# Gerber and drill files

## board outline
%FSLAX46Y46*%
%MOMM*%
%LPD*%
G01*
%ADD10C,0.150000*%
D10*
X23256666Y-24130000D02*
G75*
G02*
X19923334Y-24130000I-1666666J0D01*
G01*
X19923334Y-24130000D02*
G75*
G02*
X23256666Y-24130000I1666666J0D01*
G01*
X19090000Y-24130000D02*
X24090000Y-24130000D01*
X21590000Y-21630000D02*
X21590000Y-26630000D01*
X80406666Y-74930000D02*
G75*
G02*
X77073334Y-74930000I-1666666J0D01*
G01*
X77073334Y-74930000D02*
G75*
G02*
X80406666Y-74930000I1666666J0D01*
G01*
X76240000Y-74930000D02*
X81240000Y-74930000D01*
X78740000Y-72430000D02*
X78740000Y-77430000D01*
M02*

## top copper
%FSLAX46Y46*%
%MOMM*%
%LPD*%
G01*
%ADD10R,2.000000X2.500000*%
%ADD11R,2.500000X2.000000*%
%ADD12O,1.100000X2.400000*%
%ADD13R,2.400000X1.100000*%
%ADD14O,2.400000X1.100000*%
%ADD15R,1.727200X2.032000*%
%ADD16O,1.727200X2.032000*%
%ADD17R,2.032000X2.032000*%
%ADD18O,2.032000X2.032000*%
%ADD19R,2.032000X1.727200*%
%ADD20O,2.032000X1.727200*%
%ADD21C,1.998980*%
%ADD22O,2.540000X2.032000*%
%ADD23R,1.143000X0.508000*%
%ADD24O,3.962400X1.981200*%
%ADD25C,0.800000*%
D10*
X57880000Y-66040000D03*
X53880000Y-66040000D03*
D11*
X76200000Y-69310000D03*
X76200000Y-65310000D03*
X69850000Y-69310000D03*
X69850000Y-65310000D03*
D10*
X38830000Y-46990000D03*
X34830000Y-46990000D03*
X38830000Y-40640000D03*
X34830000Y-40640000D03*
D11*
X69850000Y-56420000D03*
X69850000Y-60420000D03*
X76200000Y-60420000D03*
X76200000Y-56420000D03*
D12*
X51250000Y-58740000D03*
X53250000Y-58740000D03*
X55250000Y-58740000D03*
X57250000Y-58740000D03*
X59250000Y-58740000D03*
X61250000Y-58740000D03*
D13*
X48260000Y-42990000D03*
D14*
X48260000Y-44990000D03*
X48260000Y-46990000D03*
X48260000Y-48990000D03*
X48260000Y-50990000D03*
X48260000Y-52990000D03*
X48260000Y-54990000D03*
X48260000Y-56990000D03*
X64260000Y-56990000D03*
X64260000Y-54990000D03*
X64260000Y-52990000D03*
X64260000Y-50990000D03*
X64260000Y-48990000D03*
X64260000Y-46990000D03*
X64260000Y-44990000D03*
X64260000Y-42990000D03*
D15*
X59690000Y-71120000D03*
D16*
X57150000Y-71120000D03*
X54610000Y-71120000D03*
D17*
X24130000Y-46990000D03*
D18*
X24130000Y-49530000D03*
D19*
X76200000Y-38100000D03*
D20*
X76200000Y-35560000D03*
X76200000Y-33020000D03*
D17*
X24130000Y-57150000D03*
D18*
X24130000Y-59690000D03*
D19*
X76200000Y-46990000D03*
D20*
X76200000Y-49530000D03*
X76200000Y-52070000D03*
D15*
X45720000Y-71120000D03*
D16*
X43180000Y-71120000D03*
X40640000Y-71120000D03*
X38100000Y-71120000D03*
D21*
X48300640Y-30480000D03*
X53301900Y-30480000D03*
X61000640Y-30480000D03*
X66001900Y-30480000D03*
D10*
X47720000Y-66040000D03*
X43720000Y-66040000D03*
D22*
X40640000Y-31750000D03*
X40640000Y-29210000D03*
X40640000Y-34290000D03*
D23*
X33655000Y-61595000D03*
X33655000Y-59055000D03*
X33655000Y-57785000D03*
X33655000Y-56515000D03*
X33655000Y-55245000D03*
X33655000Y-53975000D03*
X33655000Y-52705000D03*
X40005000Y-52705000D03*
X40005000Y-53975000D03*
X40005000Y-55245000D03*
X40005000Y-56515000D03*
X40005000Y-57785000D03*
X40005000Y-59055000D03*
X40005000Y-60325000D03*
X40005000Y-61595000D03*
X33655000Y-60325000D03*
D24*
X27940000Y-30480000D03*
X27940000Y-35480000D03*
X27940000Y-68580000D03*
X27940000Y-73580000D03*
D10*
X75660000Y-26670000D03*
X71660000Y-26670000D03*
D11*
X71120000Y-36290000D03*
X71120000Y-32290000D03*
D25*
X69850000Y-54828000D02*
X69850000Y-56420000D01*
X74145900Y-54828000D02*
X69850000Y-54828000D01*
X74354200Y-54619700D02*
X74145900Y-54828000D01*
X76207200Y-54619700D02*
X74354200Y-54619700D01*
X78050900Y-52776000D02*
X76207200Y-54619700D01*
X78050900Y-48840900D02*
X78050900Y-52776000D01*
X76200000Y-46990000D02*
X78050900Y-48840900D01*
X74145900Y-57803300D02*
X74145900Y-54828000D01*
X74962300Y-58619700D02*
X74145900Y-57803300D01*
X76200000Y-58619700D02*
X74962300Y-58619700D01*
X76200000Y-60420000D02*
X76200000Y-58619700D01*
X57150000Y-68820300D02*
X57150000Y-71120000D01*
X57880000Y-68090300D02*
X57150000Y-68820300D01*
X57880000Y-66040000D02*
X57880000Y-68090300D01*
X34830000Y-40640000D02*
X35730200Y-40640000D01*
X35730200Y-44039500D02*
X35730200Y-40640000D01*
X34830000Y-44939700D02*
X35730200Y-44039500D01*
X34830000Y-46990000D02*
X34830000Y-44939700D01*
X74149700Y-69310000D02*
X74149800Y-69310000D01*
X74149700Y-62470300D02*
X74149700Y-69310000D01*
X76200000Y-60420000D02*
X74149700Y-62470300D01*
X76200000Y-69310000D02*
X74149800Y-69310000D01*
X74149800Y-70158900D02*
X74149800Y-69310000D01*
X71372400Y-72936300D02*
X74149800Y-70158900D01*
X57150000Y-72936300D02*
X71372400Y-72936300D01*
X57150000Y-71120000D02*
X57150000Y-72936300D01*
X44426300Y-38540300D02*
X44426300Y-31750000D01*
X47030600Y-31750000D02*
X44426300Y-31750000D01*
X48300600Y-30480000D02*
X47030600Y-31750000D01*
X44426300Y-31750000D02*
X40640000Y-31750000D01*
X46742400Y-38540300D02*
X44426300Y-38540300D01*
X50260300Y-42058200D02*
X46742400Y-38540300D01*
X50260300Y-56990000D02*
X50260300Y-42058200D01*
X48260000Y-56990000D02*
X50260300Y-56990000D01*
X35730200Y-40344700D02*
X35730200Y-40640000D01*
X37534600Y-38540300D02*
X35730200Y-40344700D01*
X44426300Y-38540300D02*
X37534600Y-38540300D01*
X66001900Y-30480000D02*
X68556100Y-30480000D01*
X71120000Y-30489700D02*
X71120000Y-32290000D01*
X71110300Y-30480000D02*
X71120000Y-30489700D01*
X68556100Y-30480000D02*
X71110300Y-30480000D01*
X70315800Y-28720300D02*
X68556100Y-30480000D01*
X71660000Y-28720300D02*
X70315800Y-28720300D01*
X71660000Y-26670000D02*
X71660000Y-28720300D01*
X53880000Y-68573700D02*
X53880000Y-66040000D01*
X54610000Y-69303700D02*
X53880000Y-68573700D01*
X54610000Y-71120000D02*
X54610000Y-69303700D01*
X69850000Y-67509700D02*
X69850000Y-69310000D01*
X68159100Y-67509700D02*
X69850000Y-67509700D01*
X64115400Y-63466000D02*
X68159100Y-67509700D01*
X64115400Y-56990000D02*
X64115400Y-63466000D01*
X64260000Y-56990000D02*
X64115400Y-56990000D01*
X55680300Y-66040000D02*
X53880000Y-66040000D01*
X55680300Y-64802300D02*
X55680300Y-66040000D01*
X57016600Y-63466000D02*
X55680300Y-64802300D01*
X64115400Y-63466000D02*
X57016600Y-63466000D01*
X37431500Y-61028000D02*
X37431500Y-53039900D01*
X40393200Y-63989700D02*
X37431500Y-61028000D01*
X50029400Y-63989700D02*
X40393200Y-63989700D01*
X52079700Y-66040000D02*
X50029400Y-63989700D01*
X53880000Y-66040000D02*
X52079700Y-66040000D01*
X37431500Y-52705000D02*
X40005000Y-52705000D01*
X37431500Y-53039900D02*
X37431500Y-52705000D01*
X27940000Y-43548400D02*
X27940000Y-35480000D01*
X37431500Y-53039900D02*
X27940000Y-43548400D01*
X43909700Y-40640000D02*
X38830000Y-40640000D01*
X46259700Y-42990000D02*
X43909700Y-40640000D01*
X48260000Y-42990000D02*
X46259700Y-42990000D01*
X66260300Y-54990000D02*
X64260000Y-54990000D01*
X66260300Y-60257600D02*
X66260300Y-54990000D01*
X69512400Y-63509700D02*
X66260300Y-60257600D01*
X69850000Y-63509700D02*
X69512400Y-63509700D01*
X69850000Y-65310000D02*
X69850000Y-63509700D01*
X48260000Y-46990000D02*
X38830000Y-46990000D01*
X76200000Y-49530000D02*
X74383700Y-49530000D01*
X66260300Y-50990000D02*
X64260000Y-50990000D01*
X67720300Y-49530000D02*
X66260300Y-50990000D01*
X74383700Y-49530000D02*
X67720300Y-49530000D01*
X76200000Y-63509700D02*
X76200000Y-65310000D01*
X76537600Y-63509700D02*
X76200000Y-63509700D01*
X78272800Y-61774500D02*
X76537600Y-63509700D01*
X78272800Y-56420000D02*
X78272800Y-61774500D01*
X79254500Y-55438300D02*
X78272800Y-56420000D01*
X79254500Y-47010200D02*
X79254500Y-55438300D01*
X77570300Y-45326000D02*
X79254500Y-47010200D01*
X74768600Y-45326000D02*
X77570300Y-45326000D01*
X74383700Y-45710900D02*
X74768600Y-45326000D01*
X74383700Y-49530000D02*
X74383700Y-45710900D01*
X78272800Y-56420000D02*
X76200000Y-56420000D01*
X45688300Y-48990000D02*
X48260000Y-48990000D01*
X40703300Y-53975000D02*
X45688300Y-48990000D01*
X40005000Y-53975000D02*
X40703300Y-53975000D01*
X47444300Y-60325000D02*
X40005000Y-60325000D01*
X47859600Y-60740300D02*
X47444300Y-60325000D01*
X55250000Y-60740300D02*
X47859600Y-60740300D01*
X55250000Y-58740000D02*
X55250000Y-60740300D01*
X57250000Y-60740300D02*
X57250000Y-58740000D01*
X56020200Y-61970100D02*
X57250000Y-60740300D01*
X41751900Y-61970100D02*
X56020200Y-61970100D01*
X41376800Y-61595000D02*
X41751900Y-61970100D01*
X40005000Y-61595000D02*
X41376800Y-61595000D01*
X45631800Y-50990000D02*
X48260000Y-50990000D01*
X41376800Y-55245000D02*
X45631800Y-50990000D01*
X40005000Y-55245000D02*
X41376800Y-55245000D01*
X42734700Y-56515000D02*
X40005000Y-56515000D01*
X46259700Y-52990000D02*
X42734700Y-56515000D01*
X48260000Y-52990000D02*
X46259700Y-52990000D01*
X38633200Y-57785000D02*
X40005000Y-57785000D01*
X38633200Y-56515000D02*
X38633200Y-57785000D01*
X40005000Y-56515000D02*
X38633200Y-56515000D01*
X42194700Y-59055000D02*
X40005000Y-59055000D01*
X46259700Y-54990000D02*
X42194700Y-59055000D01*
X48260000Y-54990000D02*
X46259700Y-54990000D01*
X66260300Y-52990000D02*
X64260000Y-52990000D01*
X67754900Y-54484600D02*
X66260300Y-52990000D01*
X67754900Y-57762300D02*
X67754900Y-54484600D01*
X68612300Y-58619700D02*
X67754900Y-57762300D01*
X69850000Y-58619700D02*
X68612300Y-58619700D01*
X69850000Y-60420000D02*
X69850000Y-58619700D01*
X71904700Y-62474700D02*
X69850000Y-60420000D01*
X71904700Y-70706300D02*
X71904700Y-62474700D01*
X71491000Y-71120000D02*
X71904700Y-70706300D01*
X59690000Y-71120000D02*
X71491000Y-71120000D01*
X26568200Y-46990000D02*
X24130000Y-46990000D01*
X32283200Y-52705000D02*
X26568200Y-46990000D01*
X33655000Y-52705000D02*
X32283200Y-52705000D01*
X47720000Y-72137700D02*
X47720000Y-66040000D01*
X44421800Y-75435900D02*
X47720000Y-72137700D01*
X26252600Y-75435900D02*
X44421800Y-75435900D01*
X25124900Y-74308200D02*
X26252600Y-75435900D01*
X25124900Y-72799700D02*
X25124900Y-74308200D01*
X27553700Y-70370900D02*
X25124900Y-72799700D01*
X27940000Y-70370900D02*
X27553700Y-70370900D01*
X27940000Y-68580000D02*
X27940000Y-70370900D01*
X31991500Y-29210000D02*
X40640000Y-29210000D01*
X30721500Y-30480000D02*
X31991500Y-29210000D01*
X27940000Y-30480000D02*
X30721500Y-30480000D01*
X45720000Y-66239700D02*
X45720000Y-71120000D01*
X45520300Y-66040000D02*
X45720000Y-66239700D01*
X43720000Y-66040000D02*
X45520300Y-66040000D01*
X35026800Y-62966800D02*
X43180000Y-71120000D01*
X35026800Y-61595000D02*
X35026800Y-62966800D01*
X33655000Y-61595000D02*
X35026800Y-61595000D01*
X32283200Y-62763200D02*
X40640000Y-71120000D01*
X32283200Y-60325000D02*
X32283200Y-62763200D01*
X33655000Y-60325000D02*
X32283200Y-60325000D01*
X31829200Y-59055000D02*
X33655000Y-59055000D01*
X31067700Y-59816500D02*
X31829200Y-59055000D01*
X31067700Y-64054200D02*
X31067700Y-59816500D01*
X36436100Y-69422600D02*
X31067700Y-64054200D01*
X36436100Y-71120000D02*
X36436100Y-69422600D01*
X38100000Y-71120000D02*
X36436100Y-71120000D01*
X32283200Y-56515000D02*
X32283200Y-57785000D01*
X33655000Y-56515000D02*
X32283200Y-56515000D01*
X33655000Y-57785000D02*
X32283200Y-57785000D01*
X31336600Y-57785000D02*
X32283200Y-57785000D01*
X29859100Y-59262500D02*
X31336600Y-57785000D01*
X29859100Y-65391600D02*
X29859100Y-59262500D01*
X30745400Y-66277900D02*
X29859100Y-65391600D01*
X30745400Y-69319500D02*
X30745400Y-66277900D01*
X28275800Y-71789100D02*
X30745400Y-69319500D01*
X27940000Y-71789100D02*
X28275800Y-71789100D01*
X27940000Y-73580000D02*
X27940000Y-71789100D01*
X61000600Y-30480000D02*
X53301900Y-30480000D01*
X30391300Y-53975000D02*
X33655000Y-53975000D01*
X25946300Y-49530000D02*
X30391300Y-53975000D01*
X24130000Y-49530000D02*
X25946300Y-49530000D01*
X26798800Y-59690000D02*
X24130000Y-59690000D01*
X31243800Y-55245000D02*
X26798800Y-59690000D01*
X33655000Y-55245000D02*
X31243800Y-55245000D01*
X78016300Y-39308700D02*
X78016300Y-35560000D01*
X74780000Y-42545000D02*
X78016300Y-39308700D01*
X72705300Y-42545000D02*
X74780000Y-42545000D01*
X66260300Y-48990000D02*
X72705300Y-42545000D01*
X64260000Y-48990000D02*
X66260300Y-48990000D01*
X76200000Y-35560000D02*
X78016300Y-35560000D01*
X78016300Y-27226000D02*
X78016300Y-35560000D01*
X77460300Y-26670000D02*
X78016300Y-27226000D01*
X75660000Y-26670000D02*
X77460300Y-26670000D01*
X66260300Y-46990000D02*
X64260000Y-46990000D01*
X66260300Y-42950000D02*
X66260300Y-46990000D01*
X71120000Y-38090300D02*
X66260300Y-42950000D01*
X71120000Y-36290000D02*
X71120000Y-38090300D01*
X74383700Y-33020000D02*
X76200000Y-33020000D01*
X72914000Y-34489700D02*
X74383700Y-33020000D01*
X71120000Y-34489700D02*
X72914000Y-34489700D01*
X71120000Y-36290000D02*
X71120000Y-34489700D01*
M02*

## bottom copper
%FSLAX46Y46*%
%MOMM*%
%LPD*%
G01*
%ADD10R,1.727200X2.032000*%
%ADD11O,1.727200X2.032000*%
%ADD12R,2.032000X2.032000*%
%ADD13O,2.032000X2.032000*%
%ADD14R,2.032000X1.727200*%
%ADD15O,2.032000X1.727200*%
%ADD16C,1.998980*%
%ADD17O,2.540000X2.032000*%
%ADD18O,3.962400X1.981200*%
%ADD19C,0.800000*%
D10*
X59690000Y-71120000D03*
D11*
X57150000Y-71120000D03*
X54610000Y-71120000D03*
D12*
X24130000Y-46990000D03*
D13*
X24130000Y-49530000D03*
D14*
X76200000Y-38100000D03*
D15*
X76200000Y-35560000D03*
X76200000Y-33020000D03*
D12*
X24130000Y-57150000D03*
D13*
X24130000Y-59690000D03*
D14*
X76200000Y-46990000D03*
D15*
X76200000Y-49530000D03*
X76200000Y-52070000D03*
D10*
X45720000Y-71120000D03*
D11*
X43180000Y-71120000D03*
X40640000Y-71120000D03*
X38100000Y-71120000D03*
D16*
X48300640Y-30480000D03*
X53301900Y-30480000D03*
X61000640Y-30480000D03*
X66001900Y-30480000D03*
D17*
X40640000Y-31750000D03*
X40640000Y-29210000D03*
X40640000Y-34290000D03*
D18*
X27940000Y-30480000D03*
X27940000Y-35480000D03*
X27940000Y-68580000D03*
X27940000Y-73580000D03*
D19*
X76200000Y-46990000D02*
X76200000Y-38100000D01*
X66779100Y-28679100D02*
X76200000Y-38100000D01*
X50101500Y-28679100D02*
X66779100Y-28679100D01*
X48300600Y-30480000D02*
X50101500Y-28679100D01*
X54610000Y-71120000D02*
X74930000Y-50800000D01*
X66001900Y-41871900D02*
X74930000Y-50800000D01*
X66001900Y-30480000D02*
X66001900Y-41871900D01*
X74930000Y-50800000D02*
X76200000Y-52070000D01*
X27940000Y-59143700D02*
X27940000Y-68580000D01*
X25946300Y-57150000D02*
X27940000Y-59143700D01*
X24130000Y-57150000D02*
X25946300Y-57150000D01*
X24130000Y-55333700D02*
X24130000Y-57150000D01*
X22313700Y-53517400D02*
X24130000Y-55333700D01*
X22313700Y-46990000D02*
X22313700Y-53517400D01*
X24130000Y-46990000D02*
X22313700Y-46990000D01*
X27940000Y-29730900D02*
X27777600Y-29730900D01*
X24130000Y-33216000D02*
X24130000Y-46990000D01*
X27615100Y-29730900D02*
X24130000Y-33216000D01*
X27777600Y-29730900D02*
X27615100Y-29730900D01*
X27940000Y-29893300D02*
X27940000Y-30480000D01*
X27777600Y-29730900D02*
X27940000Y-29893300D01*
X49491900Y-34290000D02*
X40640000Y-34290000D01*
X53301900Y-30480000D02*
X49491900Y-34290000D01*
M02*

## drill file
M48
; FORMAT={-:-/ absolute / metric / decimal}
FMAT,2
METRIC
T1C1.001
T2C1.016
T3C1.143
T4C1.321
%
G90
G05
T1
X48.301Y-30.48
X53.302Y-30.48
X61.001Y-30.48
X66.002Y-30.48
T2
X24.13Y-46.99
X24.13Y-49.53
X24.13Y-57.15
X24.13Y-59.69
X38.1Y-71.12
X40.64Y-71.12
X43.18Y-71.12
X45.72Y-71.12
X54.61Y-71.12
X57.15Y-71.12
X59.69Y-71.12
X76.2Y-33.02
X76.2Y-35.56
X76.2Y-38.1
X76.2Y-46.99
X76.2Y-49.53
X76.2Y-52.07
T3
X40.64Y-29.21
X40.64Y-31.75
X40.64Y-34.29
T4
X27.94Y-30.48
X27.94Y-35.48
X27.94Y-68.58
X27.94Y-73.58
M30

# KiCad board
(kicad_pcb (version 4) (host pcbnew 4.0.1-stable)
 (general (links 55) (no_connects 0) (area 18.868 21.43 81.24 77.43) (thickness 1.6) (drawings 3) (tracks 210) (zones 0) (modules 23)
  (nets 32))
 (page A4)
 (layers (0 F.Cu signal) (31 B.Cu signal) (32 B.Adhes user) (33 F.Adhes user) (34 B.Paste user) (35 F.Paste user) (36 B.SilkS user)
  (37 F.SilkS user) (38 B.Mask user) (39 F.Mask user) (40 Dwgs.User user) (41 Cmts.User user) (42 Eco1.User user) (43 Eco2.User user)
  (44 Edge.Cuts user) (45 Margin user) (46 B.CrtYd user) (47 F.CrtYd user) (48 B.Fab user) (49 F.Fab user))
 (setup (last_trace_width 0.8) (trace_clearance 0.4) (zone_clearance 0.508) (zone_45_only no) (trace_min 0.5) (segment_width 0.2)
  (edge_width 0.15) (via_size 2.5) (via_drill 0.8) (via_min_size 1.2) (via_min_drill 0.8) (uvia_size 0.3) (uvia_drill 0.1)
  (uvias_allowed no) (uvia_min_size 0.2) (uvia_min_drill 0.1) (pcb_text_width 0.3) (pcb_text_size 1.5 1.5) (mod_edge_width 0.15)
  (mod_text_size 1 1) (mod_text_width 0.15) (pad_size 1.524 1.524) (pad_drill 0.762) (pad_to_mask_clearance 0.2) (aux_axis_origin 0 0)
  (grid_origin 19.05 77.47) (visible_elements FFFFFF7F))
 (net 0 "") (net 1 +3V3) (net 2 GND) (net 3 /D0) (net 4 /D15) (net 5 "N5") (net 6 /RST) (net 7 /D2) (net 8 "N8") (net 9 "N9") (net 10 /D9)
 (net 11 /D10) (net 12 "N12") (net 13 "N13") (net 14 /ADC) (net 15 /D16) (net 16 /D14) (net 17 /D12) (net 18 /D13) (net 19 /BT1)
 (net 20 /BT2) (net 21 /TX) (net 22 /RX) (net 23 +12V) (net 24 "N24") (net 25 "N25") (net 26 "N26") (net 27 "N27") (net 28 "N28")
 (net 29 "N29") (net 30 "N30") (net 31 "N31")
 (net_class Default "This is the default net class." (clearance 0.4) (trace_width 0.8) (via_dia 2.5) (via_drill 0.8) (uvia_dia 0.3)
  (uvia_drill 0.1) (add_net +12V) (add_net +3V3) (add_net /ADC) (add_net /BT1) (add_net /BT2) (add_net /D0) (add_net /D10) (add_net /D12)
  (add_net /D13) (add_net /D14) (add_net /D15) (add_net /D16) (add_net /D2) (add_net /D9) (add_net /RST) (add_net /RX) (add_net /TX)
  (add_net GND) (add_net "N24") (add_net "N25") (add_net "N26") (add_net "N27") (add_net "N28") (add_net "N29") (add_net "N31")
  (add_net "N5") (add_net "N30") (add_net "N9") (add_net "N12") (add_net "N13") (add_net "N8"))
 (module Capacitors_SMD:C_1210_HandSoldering (layer F.Cu) (at 55.88 66.04 180)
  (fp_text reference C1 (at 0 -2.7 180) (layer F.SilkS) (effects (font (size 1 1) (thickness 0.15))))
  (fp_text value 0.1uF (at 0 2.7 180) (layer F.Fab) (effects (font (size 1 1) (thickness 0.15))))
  (pad 1 smd rect (at -2 0 180) (size 2 2.5) (layers F.Cu F.Paste F.Mask) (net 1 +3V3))
  (pad 2 smd rect (at 2 0 180) (size 2 2.5) (layers F.Cu F.Paste F.Mask) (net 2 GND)))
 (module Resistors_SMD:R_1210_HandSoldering (layer F.Cu) (at 76.2 67.31 90)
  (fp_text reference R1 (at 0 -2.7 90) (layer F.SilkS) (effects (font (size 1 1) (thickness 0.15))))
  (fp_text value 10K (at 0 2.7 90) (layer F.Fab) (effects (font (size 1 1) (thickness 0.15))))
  (pad 1 smd rect (at -2 0 90) (size 2 2.5) (layers F.Cu F.Paste F.Mask) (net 1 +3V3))
  (pad 2 smd rect (at 2 0 90) (size 2 2.5) (layers F.Cu F.Paste F.Mask) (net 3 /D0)))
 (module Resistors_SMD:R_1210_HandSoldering (layer F.Cu) (at 69.85 67.31 90)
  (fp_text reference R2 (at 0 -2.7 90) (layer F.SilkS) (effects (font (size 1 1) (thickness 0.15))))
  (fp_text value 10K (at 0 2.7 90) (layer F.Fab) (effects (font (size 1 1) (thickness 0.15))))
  (pad 1 smd rect (at -2 0 90) (size 2 2.5) (layers F.Cu F.Paste F.Mask) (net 2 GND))
  (pad 2 smd rect (at 2 0 90) (size 2 2.5) (layers F.Cu F.Paste F.Mask) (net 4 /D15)))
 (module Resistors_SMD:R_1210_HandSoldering (layer F.Cu) (at 36.83 46.99 180)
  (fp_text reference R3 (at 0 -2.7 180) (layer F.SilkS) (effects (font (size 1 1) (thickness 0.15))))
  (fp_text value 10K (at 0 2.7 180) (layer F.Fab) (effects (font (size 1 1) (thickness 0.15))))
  (pad 1 smd rect (at -2 0 180) (size 2 2.5) (layers F.Cu F.Paste F.Mask) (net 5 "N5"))
  (pad 2 smd rect (at 2 0 180) (size 2 2.5) (layers F.Cu F.Paste F.Mask) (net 1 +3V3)))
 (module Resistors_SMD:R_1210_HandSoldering (layer F.Cu) (at 36.83 40.64 180)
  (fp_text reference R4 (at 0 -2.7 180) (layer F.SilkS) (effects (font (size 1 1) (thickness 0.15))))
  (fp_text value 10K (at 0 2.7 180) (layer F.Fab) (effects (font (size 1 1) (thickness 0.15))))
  (pad 1 smd rect (at -2 0 180) (size 2 2.5) (layers F.Cu F.Paste F.Mask) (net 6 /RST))
  (pad 2 smd rect (at 2 0 180) (size 2 2.5) (layers F.Cu F.Paste F.Mask) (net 1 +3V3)))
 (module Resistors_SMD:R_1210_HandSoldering (layer F.Cu) (at 69.85 58.42 270)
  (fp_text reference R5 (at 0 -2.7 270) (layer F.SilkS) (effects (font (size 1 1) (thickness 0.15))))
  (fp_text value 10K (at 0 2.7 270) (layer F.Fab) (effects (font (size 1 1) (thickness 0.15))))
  (pad 1 smd rect (at -2 0 270) (size 2 2.5) (layers F.Cu F.Paste F.Mask) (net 1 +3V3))
  (pad 2 smd rect (at 2 0 270) (size 2 2.5) (layers F.Cu F.Paste F.Mask) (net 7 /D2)))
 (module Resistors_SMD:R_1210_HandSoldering (layer F.Cu) (at 76.2 58.42 90)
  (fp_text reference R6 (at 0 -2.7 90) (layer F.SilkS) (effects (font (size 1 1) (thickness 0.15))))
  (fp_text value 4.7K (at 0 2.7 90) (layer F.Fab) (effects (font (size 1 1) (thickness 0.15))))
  (pad 1 smd rect (at -2 0 90) (size 2 2.5) (layers F.Cu F.Paste F.Mask) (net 1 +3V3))
  (pad 2 smd rect (at 2 0 90) (size 2 2.5) (layers F.Cu F.Paste F.Mask) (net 3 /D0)))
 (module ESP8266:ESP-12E (layer F.Cu) (at 48.26 42.99)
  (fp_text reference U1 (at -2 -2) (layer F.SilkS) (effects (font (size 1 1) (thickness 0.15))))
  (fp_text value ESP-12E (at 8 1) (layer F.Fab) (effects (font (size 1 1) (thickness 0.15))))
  (pad 9 smd oval (at 2.99 15.75 90) (size 2.4 1.1) (layers F.Cu F.Paste F.Mask) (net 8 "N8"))
  (pad 10 smd oval (at 4.99 15.75 90) (size 2.4 1.1) (layers F.Cu F.Paste F.Mask) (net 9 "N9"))
  (pad 11 smd oval (at 6.99 15.75 90) (size 2.4 1.1) (layers F.Cu F.Paste F.Mask) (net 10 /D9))
  (pad 12 smd oval (at 8.99 15.75 90) (size 2.4 1.1) (layers F.Cu F.Paste F.Mask) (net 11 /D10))
  (pad 13 smd oval (at 10.99 15.75 90) (size 2.4 1.1) (layers F.Cu F.Paste F.Mask) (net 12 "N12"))
  (pad 14 smd oval (at 12.99 15.75 90) (size 2.4 1.1) (layers F.Cu F.Paste F.Mask) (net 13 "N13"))
  (pad 1 smd rect (at 0 0) (size 2.4 1.1) (layers F.Cu F.Paste F.Mask) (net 6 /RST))
  (pad 2 smd oval (at 0 2) (size 2.4 1.1) (layers F.Cu F.Paste F.Mask) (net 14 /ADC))
  (pad 3 smd oval (at 0 4) (size 2.4 1.1) (layers F.Cu F.Paste F.Mask) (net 5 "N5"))
  (pad 4 smd oval (at 0 6) (size 2.4 1.1) (layers F.Cu F.Paste F.Mask) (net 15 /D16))
  (pad 5 smd oval (at 0 8) (size 2.4 1.1) (layers F.Cu F.Paste F.Mask) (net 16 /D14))
  (pad 6 smd oval (at 0 10) (size 2.4 1.1) (layers F.Cu F.Paste F.Mask) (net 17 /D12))
  (pad 7 smd oval (at 0 12) (size 2.4 1.1) (layers F.Cu F.Paste F.Mask) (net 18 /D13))
  (pad 8 smd oval (at 0 14) (size 2.4 1.1) (layers F.Cu F.Paste F.Mask) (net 1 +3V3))
  (pad 15 smd oval (at 16 14) (size 2.4 1.1) (layers F.Cu F.Paste F.Mask) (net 2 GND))
  (pad 16 smd oval (at 16 12) (size 2.4 1.1) (layers F.Cu F.Paste F.Mask) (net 4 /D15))
  (pad 17 smd oval (at 16 10) (size 2.4 1.1) (layers F.Cu F.Paste F.Mask) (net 7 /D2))
  (pad 18 smd oval (at 16 8) (size 2.4 1.1) (layers F.Cu F.Paste F.Mask) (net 3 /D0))
  (pad 19 smd oval (at 16 6) (size 2.4 1.1) (layers F.Cu F.Paste F.Mask) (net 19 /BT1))
  (pad 20 smd oval (at 16 4) (size 2.4 1.1) (layers F.Cu F.Paste F.Mask) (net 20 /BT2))
  (pad 21 smd oval (at 16 2) (size 2.4 1.1) (layers F.Cu F.Paste F.Mask) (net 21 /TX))
  (pad 22 smd oval (at 16 0) (size 2.4 1.1) (layers F.Cu F.Paste F.Mask) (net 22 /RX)))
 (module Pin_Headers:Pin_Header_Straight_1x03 (layer F.Cu) (at 59.69 71.12 270)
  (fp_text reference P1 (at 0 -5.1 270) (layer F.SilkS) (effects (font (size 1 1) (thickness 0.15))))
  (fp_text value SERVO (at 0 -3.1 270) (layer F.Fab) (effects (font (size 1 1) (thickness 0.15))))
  (pad 1 thru_hole rect (at 0 0 270) (size 2.032 1.7272) (drill 1.016) (layers *.Cu *.Mask F.SilkS) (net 7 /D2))
  (pad 2 thru_hole oval (at 0 2.54 270) (size 2.032 1.7272) (drill 1.016) (layers *.Cu *.Mask F.SilkS) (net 1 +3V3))
  (pad 3 thru_hole oval (at 0 5.08 270) (size 2.032 1.7272) (drill 1.016) (layers *.Cu *.Mask F.SilkS) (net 2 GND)))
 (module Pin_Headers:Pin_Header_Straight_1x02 (layer F.Cu) (at 24.13 46.99)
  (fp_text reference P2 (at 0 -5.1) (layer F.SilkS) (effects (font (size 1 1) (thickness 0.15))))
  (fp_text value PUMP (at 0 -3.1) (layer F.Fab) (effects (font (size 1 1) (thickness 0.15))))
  (pad 1 thru_hole rect (at 0 0) (size 2.032 2.032) (drill 1.016) (layers *.Cu *.Mask F.SilkS) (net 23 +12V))
  (pad 2 thru_hole oval (at 0 2.54) (size 2.032 2.032) (drill 1.016) (layers *.Cu *.Mask F.SilkS) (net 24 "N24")))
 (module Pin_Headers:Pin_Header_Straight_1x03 (layer F.Cu) (at 76.2 38.1 180)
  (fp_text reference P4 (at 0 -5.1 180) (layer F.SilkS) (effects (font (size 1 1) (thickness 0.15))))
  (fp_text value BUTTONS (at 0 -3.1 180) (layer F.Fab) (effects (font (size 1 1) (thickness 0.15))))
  (pad 1 thru_hole rect (at 0 0 180) (size 2.032 1.7272) (drill 1.016) (layers *.Cu *.Mask F.SilkS) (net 1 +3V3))
  (pad 2 thru_hole oval (at 0 2.54 180) (size 2.032 1.7272) (drill 1.016) (layers *.Cu *.Mask F.SilkS) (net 19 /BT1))
  (pad 3 thru_hole oval (at 0 5.08 180) (size 2.032 1.7272) (drill 1.016) (layers *.Cu *.Mask F.SilkS) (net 20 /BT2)))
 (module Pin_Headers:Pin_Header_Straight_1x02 (layer F.Cu) (at 24.13 57.15)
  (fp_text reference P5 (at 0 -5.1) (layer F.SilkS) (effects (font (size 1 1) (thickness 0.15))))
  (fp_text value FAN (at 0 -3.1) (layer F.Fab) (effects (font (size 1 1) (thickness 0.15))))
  (pad 1 thru_hole rect (at 0 0) (size 2.032 2.032) (drill 1.016) (layers *.Cu *.Mask F.SilkS) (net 23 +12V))
  (pad 2 thru_hole oval (at 0 2.54) (size 2.032 2.032) (drill 1.016) (layers *.Cu *.Mask F.SilkS) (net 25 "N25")))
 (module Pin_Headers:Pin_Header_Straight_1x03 (layer F.Cu) (at 76.2 46.99)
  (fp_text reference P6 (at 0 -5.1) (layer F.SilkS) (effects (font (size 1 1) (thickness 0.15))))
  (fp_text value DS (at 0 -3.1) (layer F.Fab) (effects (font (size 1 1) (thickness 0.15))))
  (pad 1 thru_hole rect (at 0 0) (size 2.032 1.7272) (drill 1.016) (layers *.Cu *.Mask F.SilkS) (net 1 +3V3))
  (pad 2 thru_hole oval (at 0 2.54) (size 2.032 1.7272) (drill 1.016) (layers *.Cu *.Mask F.SilkS) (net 3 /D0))
  (pad 3 thru_hole oval (at 0 5.08) (size 2.032 1.7272) (drill 1.016) (layers *.Cu *.Mask F.SilkS) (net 2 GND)))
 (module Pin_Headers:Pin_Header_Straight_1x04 (layer F.Cu) (at 45.72 71.12 270)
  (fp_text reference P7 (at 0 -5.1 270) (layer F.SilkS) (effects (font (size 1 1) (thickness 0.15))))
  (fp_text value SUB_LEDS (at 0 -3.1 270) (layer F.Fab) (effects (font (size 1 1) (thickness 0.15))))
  (pad 1 thru_hole rect (at 0 0 270) (size 2.032 1.7272) (drill 1.016) (layers *.Cu *.Mask F.SilkS) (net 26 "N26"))
  (pad 2 thru_hole oval (at 0 2.54 270) (size 2.032 1.7272) (drill 1.016) (layers *.Cu *.Mask F.SilkS) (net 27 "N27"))
  (pad 3 thru_hole oval (at 0 5.08 270) (size 2.032 1.7272) (drill 1.016) (layers *.Cu *.Mask F.SilkS) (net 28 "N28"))
  (pad 4 thru_hole oval (at 0 7.62 270) (size 2.032 1.7272) (drill 1.016) (layers *.Cu *.Mask F.SilkS) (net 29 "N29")))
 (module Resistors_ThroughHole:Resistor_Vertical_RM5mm (layer F.Cu) (at 50.8 30.48)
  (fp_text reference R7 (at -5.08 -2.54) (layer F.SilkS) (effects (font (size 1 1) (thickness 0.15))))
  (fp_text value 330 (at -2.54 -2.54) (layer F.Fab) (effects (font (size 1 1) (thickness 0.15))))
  (pad 1 thru_hole circle (at -2.49936 0) (size 1.99898 1.99898) (drill 1.00076) (layers *.Cu *.SilkS *.Mask) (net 1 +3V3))
  (pad 2 thru_hole circle (at 2.5019 0) (size 1.99898 1.99898) (drill 1.00076) (layers *.Cu *.SilkS *.Mask) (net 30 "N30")))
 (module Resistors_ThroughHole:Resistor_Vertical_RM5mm (layer F.Cu) (at 63.5 30.48)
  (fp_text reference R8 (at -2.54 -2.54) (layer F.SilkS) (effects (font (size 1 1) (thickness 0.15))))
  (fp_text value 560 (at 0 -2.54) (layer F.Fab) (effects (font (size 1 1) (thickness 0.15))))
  (pad 1 thru_hole circle (at -2.49936 0) (size 1.99898 1.99898) (drill 1.00076) (layers *.Cu *.SilkS *.Mask) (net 30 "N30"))
  (pad 2 thru_hole circle (at 2.5019 0) (size 1.99898 1.99898) (drill 1.00076) (layers *.Cu *.SilkS *.Mask) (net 2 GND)))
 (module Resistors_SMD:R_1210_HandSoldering (layer F.Cu) (at 45.72 66.04 180)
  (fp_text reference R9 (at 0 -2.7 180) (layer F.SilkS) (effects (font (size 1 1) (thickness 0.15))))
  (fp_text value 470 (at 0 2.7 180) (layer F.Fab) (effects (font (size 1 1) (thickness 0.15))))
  (pad 1 smd rect (at -2 0 180) (size 2 2.5) (layers F.Cu F.Paste F.Mask) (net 23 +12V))
  (pad 2 smd rect (at 2 0 180) (size 2 2.5) (layers F.Cu F.Paste F.Mask) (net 26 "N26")))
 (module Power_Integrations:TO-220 (layer F.Cu) (at 40.64 31.75 90)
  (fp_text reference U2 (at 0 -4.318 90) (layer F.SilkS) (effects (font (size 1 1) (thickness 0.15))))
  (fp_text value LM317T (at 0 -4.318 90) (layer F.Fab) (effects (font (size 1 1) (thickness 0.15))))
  (pad 2 thru_hole oval (at 0 0 90) (size 2.032 2.54) (drill 1.143) (layers *.Cu *.Mask F.SilkS) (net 1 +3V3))
  (pad 3 thru_hole oval (at 2.54 0 90) (size 2.032 2.54) (drill 1.143) (layers *.Cu *.Mask F.SilkS) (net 23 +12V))
  (pad 1 thru_hole oval (at -2.54 0 90) (size 2.032 2.54) (drill 1.143) (layers *.Cu *.Mask F.SilkS) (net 30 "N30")))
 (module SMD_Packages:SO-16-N (layer F.Cu) (at 36.83 57.15 90)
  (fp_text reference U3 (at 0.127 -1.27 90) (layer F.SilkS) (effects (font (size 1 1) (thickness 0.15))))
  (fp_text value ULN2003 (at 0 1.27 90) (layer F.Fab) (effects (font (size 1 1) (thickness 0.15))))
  (pad 16 smd rect (at -4.445 -3.175 90) (size 0.508 1.143) (layers F.Cu F.Paste F.Mask) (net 27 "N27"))
  (pad 14 smd rect (at -1.905 -3.175 90) (size 0.508 1.143) (layers F.Cu F.Paste F.Mask) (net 29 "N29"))
  (pad 13 smd rect (at -0.635 -3.175 90) (size 0.508 1.143) (layers F.Cu F.Paste F.Mask) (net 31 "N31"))
  (pad 12 smd rect (at 0.635 -3.175 90) (size 0.508 1.143) (layers F.Cu F.Paste F.Mask) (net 31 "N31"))
  (pad 11 smd rect (at 1.905 -3.175 90) (size 0.508 1.143) (layers F.Cu F.Paste F.Mask) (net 25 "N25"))
  (pad 10 smd rect (at 3.175 -3.175 90) (size 0.508 1.143) (layers F.Cu F.Paste F.Mask) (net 24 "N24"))
  (pad 9 smd rect (at 4.445 -3.175 90) (size 0.508 1.143) (layers F.Cu F.Paste F.Mask) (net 23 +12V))
  (pad 8 smd rect (at 4.445 3.175 90) (size 0.508 1.143) (layers F.Cu F.Paste F.Mask) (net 2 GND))
  (pad 7 smd rect (at 3.175 3.175 90) (size 0.508 1.143) (layers F.Cu F.Paste F.Mask) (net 15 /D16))
  (pad 6 smd rect (at 1.905 3.175 90) (size 0.508 1.143) (layers F.Cu F.Paste F.Mask) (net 16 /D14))
  (pad 5 smd rect (at 0.635 3.175 90) (size 0.508 1.143) (layers F.Cu F.Paste F.Mask) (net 17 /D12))
  (pad 4 smd rect (at -0.635 3.175 90) (size 0.508 1.143) (layers F.Cu F.Paste F.Mask) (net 17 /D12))
  (pad 3 smd rect (at -1.905 3.175 90) (size 0.508 1.143) (layers F.Cu F.Paste F.Mask) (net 18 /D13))
  (pad 2 smd rect (at -3.175 3.175 90) (size 0.508 1.143) (layers F.Cu F.Paste F.Mask) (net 10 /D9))
  (pad 1 smd rect (at -4.445 3.175 90) (size 0.508 1.143) (layers F.Cu F.Paste F.Mask) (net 11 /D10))
  (pad 15 smd rect (at -3.175 -3.175 90) (size 0.508 1.143) (layers F.Cu F.Paste F.Mask) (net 28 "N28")))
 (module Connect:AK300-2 (layer F.Cu) (at 27.94 30.48 270)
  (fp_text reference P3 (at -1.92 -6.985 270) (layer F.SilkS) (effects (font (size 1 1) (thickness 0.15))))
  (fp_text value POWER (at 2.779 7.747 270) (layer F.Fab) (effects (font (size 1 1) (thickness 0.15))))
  (pad 1 thru_hole oval (at 0 0 270) (size 1.9812 3.9624) (drill 1.3208) (layers *.Cu F.Paste F.SilkS F.Mask) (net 23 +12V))
  (pad 2 thru_hole oval (at 5 0 270) (size 1.9812 3.9624) (drill 1.3208) (layers *.Cu F.Paste F.SilkS F.Mask) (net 2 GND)))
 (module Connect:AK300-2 (layer F.Cu) (at 27.94 68.58 270)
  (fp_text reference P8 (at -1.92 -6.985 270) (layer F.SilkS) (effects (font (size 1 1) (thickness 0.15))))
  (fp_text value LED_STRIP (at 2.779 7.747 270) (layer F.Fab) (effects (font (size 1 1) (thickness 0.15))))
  (pad 1 thru_hole oval (at 0 0 270) (size 1.9812 3.9624) (drill 1.3208) (layers *.Cu F.Paste F.SilkS F.Mask) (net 23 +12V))
  (pad 2 thru_hole oval (at 5 0 270) (size 1.9812 3.9624) (drill 1.3208) (layers *.Cu F.Paste F.SilkS F.Mask) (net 31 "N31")))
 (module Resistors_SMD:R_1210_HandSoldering (layer F.Cu) (at 73.66 26.67 180)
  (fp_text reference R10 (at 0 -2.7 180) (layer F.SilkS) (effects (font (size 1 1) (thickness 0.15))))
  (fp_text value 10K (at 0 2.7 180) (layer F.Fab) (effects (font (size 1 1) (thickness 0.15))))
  (pad 1 smd rect (at -2 0 180) (size 2 2.5) (layers F.Cu F.Paste F.Mask) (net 19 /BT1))
  (pad 2 smd rect (at 2 0 180) (size 2 2.5) (layers F.Cu F.Paste F.Mask) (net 2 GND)))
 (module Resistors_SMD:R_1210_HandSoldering (layer F.Cu) (at 71.12 34.29 90)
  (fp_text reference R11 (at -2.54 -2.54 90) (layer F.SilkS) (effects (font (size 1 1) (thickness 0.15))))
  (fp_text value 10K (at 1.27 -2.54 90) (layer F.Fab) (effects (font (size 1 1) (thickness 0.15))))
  (pad 1 smd rect (at -2 0 90) (size 2 2.5) (layers F.Cu F.Paste F.Mask) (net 20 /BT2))
  (pad 2 smd rect (at 2 0 90) (size 2 2.5) (layers F.Cu F.Paste F.Mask) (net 2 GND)))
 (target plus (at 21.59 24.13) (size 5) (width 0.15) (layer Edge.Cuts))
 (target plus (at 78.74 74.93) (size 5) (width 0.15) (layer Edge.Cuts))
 (segment (start 76.2 46.99) (end 76.2 38.1) (width 0.8) (layer B.Cu) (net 1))
 (segment (start 69.85 54.828) (end 69.85 56.42) (width 0.8) (layer F.Cu) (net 1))
 (segment (start 74.1459 54.828) (end 69.85 54.828) (width 0.8) (layer F.Cu) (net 1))
 (segment (start 74.3542 54.6197) (end 74.1459 54.828) (width 0.8) (layer F.Cu) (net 1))
 (segment (start 76.2072 54.6197) (end 74.3542 54.6197) (width 0.8) (layer F.Cu) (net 1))
 (segment (start 78.0509 52.776) (end 76.2072 54.6197) (width 0.8) (layer F.Cu) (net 1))
 (segment (start 78.0509 48.8409) (end 78.0509 52.776) (width 0.8) (layer F.Cu) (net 1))
 (segment (start 76.2 46.99) (end 78.0509 48.8409) (width 0.8) (layer F.Cu) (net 1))
 (segment (start 74.1459 57.8033) (end 74.1459 54.828) (width 0.8) (layer F.Cu) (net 1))
 (segment (start 74.9623 58.6197) (end 74.1459 57.8033) (width 0.8) (layer F.Cu) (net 1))
 (segment (start 76.2 58.6197) (end 74.9623 58.6197) (width 0.8) (layer F.Cu) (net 1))
 (segment (start 76.2 60.42) (end 76.2 58.6197) (width 0.8) (layer F.Cu) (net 1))
 (segment (start 66.7791 28.6791) (end 76.2 38.1) (width 0.8) (layer B.Cu) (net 1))
 (segment (start 50.1015 28.6791) (end 66.7791 28.6791) (width 0.8) (layer B.Cu) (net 1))
 (segment (start 48.3006 30.48) (end 50.1015 28.6791) (width 0.8) (layer B.Cu) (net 1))
 (segment (start 57.15 68.8203) (end 57.15 71.12) (width 0.8) (layer F.Cu) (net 1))
 (segment (start 57.88 68.0903) (end 57.15 68.8203) (width 0.8) (layer F.Cu) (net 1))
 (segment (start 57.88 66.04) (end 57.88 68.0903) (width 0.8) (layer F.Cu) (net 1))
 (segment (start 34.83 40.64) (end 35.7302 40.64) (width 0.8) (layer F.Cu) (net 1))
 (segment (start 35.7302 44.0395) (end 35.7302 40.64) (width 0.8) (layer F.Cu) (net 1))
 (segment (start 34.83 44.9397) (end 35.7302 44.0395) (width 0.8) (layer F.Cu) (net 1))
 (segment (start 34.83 46.99) (end 34.83 44.9397) (width 0.8) (layer F.Cu) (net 1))
 (segment (start 74.1497 69.31) (end 74.1498 69.31) (width 0.8) (layer F.Cu) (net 1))
 (segment (start 74.1497 62.4703) (end 74.1497 69.31) (width 0.8) (layer F.Cu) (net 1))
 (segment (start 76.2 60.42) (end 74.1497 62.4703) (width 0.8) (layer F.Cu) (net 1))
 (segment (start 76.2 69.31) (end 74.1498 69.31) (width 0.8) (layer F.Cu) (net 1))
 (segment (start 74.1498 70.1589) (end 74.1498 69.31) (width 0.8) (layer F.Cu) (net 1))
 (segment (start 71.3724 72.9363) (end 74.1498 70.1589) (width 0.8) (layer F.Cu) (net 1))
 (segment (start 57.15 72.9363) (end 71.3724 72.9363) (width 0.8) (layer F.Cu) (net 1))
 (segment (start 57.15 71.12) (end 57.15 72.9363) (width 0.8) (layer F.Cu) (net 1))
 (segment (start 44.4263 38.5403) (end 44.4263 31.75) (width 0.8) (layer F.Cu) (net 1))
 (segment (start 47.0306 31.75) (end 44.4263 31.75) (width 0.8) (layer F.Cu) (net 1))
 (segment (start 48.3006 30.48) (end 47.0306 31.75) (width 0.8) (layer F.Cu) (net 1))
 (segment (start 44.4263 31.75) (end 40.64 31.75) (width 0.8) (layer F.Cu) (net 1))
 (segment (start 46.7424 38.5403) (end 44.4263 38.5403) (width 0.8) (layer F.Cu) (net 1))
 (segment (start 50.2603 42.0582) (end 46.7424 38.5403) (width 0.8) (layer F.Cu) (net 1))
 (segment (start 50.2603 56.99) (end 50.2603 42.0582) (width 0.8) (layer F.Cu) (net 1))
 (segment (start 48.26 56.99) (end 50.2603 56.99) (width 0.8) (layer F.Cu) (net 1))
 (segment (start 35.7302 40.3447) (end 35.7302 40.64) (width 0.8) (layer F.Cu) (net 1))
 (segment (start 37.5346 38.5403) (end 35.7302 40.3447) (width 0.8) (layer F.Cu) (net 1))
 (segment (start 44.4263 38.5403) (end 37.5346 38.5403) (width 0.8) (layer F.Cu) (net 1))
 (segment (start 66.0019 30.48) (end 68.5561 30.48) (width 0.8) (layer F.Cu) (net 2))
 (segment (start 71.12 30.4897) (end 71.12 32.29) (width 0.8) (layer F.Cu) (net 2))
 (segment (start 71.1103 30.48) (end 71.12 30.4897) (width 0.8) (layer F.Cu) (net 2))
 (segment (start 68.5561 30.48) (end 71.1103 30.48) (width 0.8) (layer F.Cu) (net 2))
 (segment (start 70.3158 28.7203) (end 68.5561 30.48) (width 0.8) (layer F.Cu) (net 2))
 (segment (start 71.66 28.7203) (end 70.3158 28.7203) (width 0.8) (layer F.Cu) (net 2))
 (segment (start 71.66 26.67) (end 71.66 28.7203) (width 0.8) (layer F.Cu) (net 2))
 (segment (start 53.88 68.5737) (end 53.88 66.04) (width 0.8) (layer F.Cu) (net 2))
 (segment (start 54.61 69.3037) (end 53.88 68.5737) (width 0.8) (layer F.Cu) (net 2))
 (segment (start 54.61 71.12) (end 54.61 69.3037) (width 0.8) (layer F.Cu) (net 2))
 (segment (start 69.85 67.5097) (end 69.85 69.31) (width 0.8) (layer F.Cu) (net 2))
 (segment (start 68.1591 67.5097) (end 69.85 67.5097) (width 0.8) (layer F.Cu) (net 2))
 (segment (start 64.1154 63.466) (end 68.1591 67.5097) (width 0.8) (layer F.Cu) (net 2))
 (segment (start 64.1154 56.99) (end 64.1154 63.466) (width 0.8) (layer F.Cu) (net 2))
 (segment (start 64.26 56.99) (end 64.1154 56.99) (width 0.8) (layer F.Cu) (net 2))
 (segment (start 55.6803 66.04) (end 53.88 66.04) (width 0.8) (layer F.Cu) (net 2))
 (segment (start 55.6803 64.8023) (end 55.6803 66.04) (width 0.8) (layer F.Cu) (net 2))
 (segment (start 57.0166 63.466) (end 55.6803 64.8023) (width 0.8) (layer F.Cu) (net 2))
 (segment (start 64.1154 63.466) (end 57.0166 63.466) (width 0.8) (layer F.Cu) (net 2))
 (segment (start 54.61 71.12) (end 74.93 50.8) (width 0.8) (layer B.Cu) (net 2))
 (segment (start 66.0019 41.8719) (end 74.93 50.8) (width 0.8) (layer B.Cu) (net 2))
 (segment (start 66.0019 30.48) (end 66.0019 41.8719) (width 0.8) (layer B.Cu) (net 2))
 (segment (start 74.93 50.8) (end 76.2 52.07) (width 0.8) (layer B.Cu) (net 2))
 (segment (start 37.4315 61.028) (end 37.4315 53.0399) (width 0.8) (layer F.Cu) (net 2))
 (segment (start 40.3932 63.9897) (end 37.4315 61.028) (width 0.8) (layer F.Cu) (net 2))
 (segment (start 50.0294 63.9897) (end 40.3932 63.9897) (width 0.8) (layer F.Cu) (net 2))
 (segment (start 52.0797 66.04) (end 50.0294 63.9897) (width 0.8) (layer F.Cu) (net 2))
 (segment (start 53.88 66.04) (end 52.0797 66.04) (width 0.8) (layer F.Cu) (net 2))
 (segment (start 37.4315 52.705) (end 40.005 52.705) (width 0.8) (layer F.Cu) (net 2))
 (segment (start 37.4315 53.0399) (end 37.4315 52.705) (width 0.8) (layer F.Cu) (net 2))
 (segment (start 27.94 43.5484) (end 27.94 35.48) (width 0.8) (layer F.Cu) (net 2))
 (segment (start 37.4315 53.0399) (end 27.94 43.5484) (width 0.8) (layer F.Cu) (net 2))
 (segment (start 43.9097 40.64) (end 38.83 40.64) (width 0.8) (layer F.Cu) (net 6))
 (segment (start 46.2597 42.99) (end 43.9097 40.64) (width 0.8) (layer F.Cu) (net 6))
 (segment (start 48.26 42.99) (end 46.2597 42.99) (width 0.8) (layer F.Cu) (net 6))
 (segment (start 66.2603 54.99) (end 64.26 54.99) (width 0.8) (layer F.Cu) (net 4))
 (segment (start 66.2603 60.2576) (end 66.2603 54.99) (width 0.8) (layer F.Cu) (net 4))
 (segment (start 69.5124 63.5097) (end 66.2603 60.2576) (width 0.8) (layer F.Cu) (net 4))
 (segment (start 69.85 63.5097) (end 69.5124 63.5097) (width 0.8) (layer F.Cu) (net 4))
 (segment (start 69.85 65.31) (end 69.85 63.5097) (width 0.8) (layer F.Cu) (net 4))
 (segment (start 48.26 46.99) (end 38.83 46.99) (width 0.8) (layer F.Cu) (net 5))
 (segment (start 76.2 49.53) (end 74.3837 49.53) (width 0.8) (layer F.Cu) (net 3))
 (segment (start 66.2603 50.99) (end 64.26 50.99) (width 0.8) (layer F.Cu) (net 3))
 (segment (start 67.7203 49.53) (end 66.2603 50.99) (width 0.8) (layer F.Cu) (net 3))
 (segment (start 74.3837 49.53) (end 67.7203 49.53) (width 0.8) (layer F.Cu) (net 3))
 (segment (start 76.2 63.5097) (end 76.2 65.31) (width 0.8) (layer F.Cu) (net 3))
 (segment (start 76.5376 63.5097) (end 76.2 63.5097) (width 0.8) (layer F.Cu) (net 3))
 (segment (start 78.2728 61.7745) (end 76.5376 63.5097) (width 0.8) (layer F.Cu) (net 3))
 (segment (start 78.2728 56.42) (end 78.2728 61.7745) (width 0.8) (layer F.Cu) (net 3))
 (segment (start 79.2545 55.4383) (end 78.2728 56.42) (width 0.8) (layer F.Cu) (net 3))
 (segment (start 79.2545 47.0102) (end 79.2545 55.4383) (width 0.8) (layer F.Cu) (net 3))
 (segment (start 77.5703 45.326) (end 79.2545 47.0102) (width 0.8) (layer F.Cu) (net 3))
 (segment (start 74.7686 45.326) (end 77.5703 45.326) (width 0.8) (layer F.Cu) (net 3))
 (segment (start 74.3837 45.7109) (end 74.7686 45.326) (width 0.8) (layer F.Cu) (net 3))
 (segment (start 74.3837 49.53) (end 74.3837 45.7109) (width 0.8) (layer F.Cu) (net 3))
 (segment (start 78.2728 56.42) (end 76.2 56.42) (width 0.8) (layer F.Cu) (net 3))
 (segment (start 45.6883 48.99) (end 48.26 48.99) (width 0.8) (layer F.Cu) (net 15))
 (segment (start 40.7033 53.975) (end 45.6883 48.99) (width 0.8) (layer F.Cu) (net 15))
 (segment (start 40.005 53.975) (end 40.7033 53.975) (width 0.8) (layer F.Cu) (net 15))
 (segment (start 47.4443 60.325) (end 40.005 60.325) (width 0.8) (layer F.Cu) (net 10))
 (segment (start 47.8596 60.7403) (end 47.4443 60.325) (width 0.8) (layer F.Cu) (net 10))
 (segment (start 55.25 60.7403) (end 47.8596 60.7403) (width 0.8) (layer F.Cu) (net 10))
 (segment (start 55.25 58.74) (end 55.25 60.7403) (width 0.8) (layer F.Cu) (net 10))
 (segment (start 57.25 60.7403) (end 57.25 58.74) (width 0.8) (layer F.Cu) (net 11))
 (segment (start 56.0202 61.9701) (end 57.25 60.7403) (width 0.8) (layer F.Cu) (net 11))
 (segment (start 41.7519 61.9701) (end 56.0202 61.9701) (width 0.8) (layer F.Cu) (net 11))
 (segment (start 41.3768 61.595) (end 41.7519 61.9701) (width 0.8) (layer F.Cu) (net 11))
 (segment (start 40.005 61.595) (end 41.3768 61.595) (width 0.8) (layer F.Cu) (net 11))
 (segment (start 45.6318 50.99) (end 48.26 50.99) (width 0.8) (layer F.Cu) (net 16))
 (segment (start 41.3768 55.245) (end 45.6318 50.99) (width 0.8) (layer F.Cu) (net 16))
 (segment (start 40.005 55.245) (end 41.3768 55.245) (width 0.8) (layer F.Cu) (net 16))
 (segment (start 42.7347 56.515) (end 40.005 56.515) (width 0.8) (layer F.Cu) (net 17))
 (segment (start 46.2597 52.99) (end 42.7347 56.515) (width 0.8) (layer F.Cu) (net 17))
 (segment (start 48.26 52.99) (end 46.2597 52.99) (width 0.8) (layer F.Cu) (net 17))
 (segment (start 38.6332 57.785) (end 40.005 57.785) (width 0.8) (layer F.Cu) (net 17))
 (segment (start 38.6332 56.515) (end 38.6332 57.785) (width 0.8) (layer F.Cu) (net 17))
 (segment (start 40.005 56.515) (end 38.6332 56.515) (width 0.8) (layer F.Cu) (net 17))
 (segment (start 42.1947 59.055) (end 40.005 59.055) (width 0.8) (layer F.Cu) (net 18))
 (segment (start 46.2597 54.99) (end 42.1947 59.055) (width 0.8) (layer F.Cu) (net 18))
 (segment (start 48.26 54.99) (end 46.2597 54.99) (width 0.8) (layer F.Cu) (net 18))
 (segment (start 66.2603 52.99) (end 64.26 52.99) (width 0.8) (layer F.Cu) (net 7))
 (segment (start 67.7549 54.4846) (end 66.2603 52.99) (width 0.8) (layer F.Cu) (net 7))
 (segment (start 67.7549 57.7623) (end 67.7549 54.4846) (width 0.8) (layer F.Cu) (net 7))
 (segment (start 68.6123 58.6197) (end 67.7549 57.7623) (width 0.8) (layer F.Cu) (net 7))
 (segment (start 69.85 58.6197) (end 68.6123 58.6197) (width 0.8) (layer F.Cu) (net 7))
 (segment (start 69.85 60.42) (end 69.85 58.6197) (width 0.8) (layer F.Cu) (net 7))
 (segment (start 71.9047 62.4747) (end 69.85 60.42) (width 0.8) (layer F.Cu) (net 7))
 (segment (start 71.9047 70.7063) (end 71.9047 62.4747) (width 0.8) (layer F.Cu) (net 7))
 (segment (start 71.491 71.12) (end 71.9047 70.7063) (width 0.8) (layer F.Cu) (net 7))
 (segment (start 59.69 71.12) (end 71.491 71.12) (width 0.8) (layer F.Cu) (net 7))
 (segment (start 26.5682 46.99) (end 24.13 46.99) (width 0.8) (layer F.Cu) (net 23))
 (segment (start 32.2832 52.705) (end 26.5682 46.99) (width 0.8) (layer F.Cu) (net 23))
 (segment (start 33.655 52.705) (end 32.2832 52.705) (width 0.8) (layer F.Cu) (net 23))
 (segment (start 47.72 72.1377) (end 47.72 66.04) (width 0.8) (layer F.Cu) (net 23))
 (segment (start 44.4218 75.4359) (end 47.72 72.1377) (width 0.8) (layer F.Cu) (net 23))
 (segment (start 26.2526 75.4359) (end 44.4218 75.4359) (width 0.8) (layer F.Cu) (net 23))
 (segment (start 25.1249 74.3082) (end 26.2526 75.4359) (width 0.8) (layer F.Cu) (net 23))
 (segment (start 25.1249 72.7997) (end 25.1249 74.3082) (width 0.8) (layer F.Cu) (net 23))
 (segment (start 27.5537 70.3709) (end 25.1249 72.7997) (width 0.8) (layer F.Cu) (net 23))
 (segment (start 27.94 70.3709) (end 27.5537 70.3709) (width 0.8) (layer F.Cu) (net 23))
 (segment (start 27.94 68.58) (end 27.94 70.3709) (width 0.8) (layer F.Cu) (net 23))
 (segment (start 27.94 59.1437) (end 27.94 68.58) (width 0.8) (layer B.Cu) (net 23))
 (segment (start 25.9463 57.15) (end 27.94 59.1437) (width 0.8) (layer B.Cu) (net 23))
 (segment (start 24.13 57.15) (end 25.9463 57.15) (width 0.8) (layer B.Cu) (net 23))
 (segment (start 24.13 55.3337) (end 24.13 57.15) (width 0.8) (layer B.Cu) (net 23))
 (segment (start 22.3137 53.5174) (end 24.13 55.3337) (width 0.8) (layer B.Cu) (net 23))
 (segment (start 22.3137 46.99) (end 22.3137 53.5174) (width 0.8) (layer B.Cu) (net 23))
 (segment (start 24.13 46.99) (end 22.3137 46.99) (width 0.8) (layer B.Cu) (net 23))
 (segment (start 27.94 29.7309) (end 27.7776 29.7309) (width 0.8) (layer B.Cu) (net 23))
 (segment (start 24.13 33.216) (end 24.13 46.99) (width 0.8) (layer B.Cu) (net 23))
 (segment (start 27.6151 29.7309) (end 24.13 33.216) (width 0.8) (layer B.Cu) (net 23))
 (segment (start 27.7776 29.7309) (end 27.6151 29.7309) (width 0.8) (layer B.Cu) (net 23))
 (segment (start 27.94 29.8933) (end 27.94 30.48) (width 0.8) (layer B.Cu) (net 23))
 (segment (start 27.7776 29.7309) (end 27.94 29.8933) (width 0.8) (layer B.Cu) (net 23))
 (segment (start 31.9915 29.21) (end 40.64 29.21) (width 0.8) (layer F.Cu) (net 23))
 (segment (start 30.7215 30.48) (end 31.9915 29.21) (width 0.8) (layer F.Cu) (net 23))
 (segment (start 27.94 30.48) (end 30.7215 30.48) (width 0.8) (layer F.Cu) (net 23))
 (segment (start 45.72 66.2397) (end 45.72 71.12) (width 0.8) (layer F.Cu) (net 26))
 (segment (start 45.5203 66.04) (end 45.72 66.2397) (width 0.8) (layer F.Cu) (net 26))
 (segment (start 43.72 66.04) (end 45.5203 66.04) (width 0.8) (layer F.Cu) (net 26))
 (segment (start 35.0268 62.9668) (end 43.18 71.12) (width 0.8) (layer F.Cu) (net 27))
 (segment (start 35.0268 61.595) (end 35.0268 62.9668) (width 0.8) (layer F.Cu) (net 27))
 (segment (start 33.655 61.595) (end 35.0268 61.595) (width 0.8) (layer F.Cu) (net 27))
 (segment (start 32.2832 62.7632) (end 40.64 71.12) (width 0.8) (layer F.Cu) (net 28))
 (segment (start 32.2832 60.325) (end 32.2832 62.7632) (width 0.8) (layer F.Cu) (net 28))
 (segment (start 33.655 60.325) (end 32.2832 60.325) (width 0.8) (layer F.Cu) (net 28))
 (segment (start 31.8292 59.055) (end 33.655 59.055) (width 0.8) (layer F.Cu) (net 29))
 (segment (start 31.0677 59.8165) (end 31.8292 59.055) (width 0.8) (layer F.Cu) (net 29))
 (segment (start 31.0677 64.0542) (end 31.0677 59.8165) (width 0.8) (layer F.Cu) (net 29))
 (segment (start 36.4361 69.4226) (end 31.0677 64.0542) (width 0.8) (layer F.Cu) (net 29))
 (segment (start 36.4361 71.12) (end 36.4361 69.4226) (width 0.8) (layer F.Cu) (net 29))
 (segment (start 38.1 71.12) (end 36.4361 71.12) (width 0.8) (layer F.Cu) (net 29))
 (segment (start 32.2832 56.515) (end 32.2832 57.785) (width 0.8) (layer F.Cu) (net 31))
 (segment (start 33.655 56.515) (end 32.2832 56.515) (width 0.8) (layer F.Cu) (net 31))
 (segment (start 33.655 57.785) (end 32.2832 57.785) (width 0.8) (layer F.Cu) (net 31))
 (segment (start 31.3366 57.785) (end 32.2832 57.785) (width 0.8) (layer F.Cu) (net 31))
 (segment (start 29.8591 59.2625) (end 31.3366 57.785) (width 0.8) (layer F.Cu) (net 31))
 (segment (start 29.8591 65.3916) (end 29.8591 59.2625) (width 0.8) (layer F.Cu) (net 31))
 (segment (start 30.7454 66.2779) (end 29.8591 65.3916) (width 0.8) (layer F.Cu) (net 31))
 (segment (start 30.7454 69.3195) (end 30.7454 66.2779) (width 0.8) (layer F.Cu) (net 31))
 (segment (start 28.2758 71.7891) (end 30.7454 69.3195) (width 0.8) (layer F.Cu) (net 31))
 (segment (start 27.94 71.7891) (end 28.2758 71.7891) (width 0.8) (layer F.Cu) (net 31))
 (segment (start 27.94 73.58) (end 27.94 71.7891) (width 0.8) (layer F.Cu) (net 31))
 (segment (start 61.0006 30.48) (end 53.3019 30.48) (width 0.8) (layer F.Cu) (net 30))
 (segment (start 49.4919 34.29) (end 40.64 34.29) (width 0.8) (layer B.Cu) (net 30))
 (segment (start 53.3019 30.48) (end 49.4919 34.29) (width 0.8) (layer B.Cu) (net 30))
 (segment (start 30.3913 53.975) (end 33.655 53.975) (width 0.8) (layer F.Cu) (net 24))
 (segment (start 25.9463 49.53) (end 30.3913 53.975) (width 0.8) (layer F.Cu) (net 24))
 (segment (start 24.13 49.53) (end 25.9463 49.53) (width 0.8) (layer F.Cu) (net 24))
 (segment (start 26.7988 59.69) (end 24.13 59.69) (width 0.8) (layer F.Cu) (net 25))
 (segment (start 31.2438 55.245) (end 26.7988 59.69) (width 0.8) (layer F.Cu) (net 25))
 (segment (start 33.655 55.245) (end 31.2438 55.245) (width 0.8) (layer F.Cu) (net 25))
 (segment (start 78.0163 39.3087) (end 78.0163 35.56) (width 0.8) (layer F.Cu) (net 19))
 (segment (start 74.78 42.545) (end 78.0163 39.3087) (width 0.8) (layer F.Cu) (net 19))
 (segment (start 72.7053 42.545) (end 74.78 42.545) (width 0.8) (layer F.Cu) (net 19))
 (segment (start 66.2603 48.99) (end 72.7053 42.545) (width 0.8) (layer F.Cu) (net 19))
 (segment (start 64.26 48.99) (end 66.2603 48.99) (width 0.8) (layer F.Cu) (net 19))
 (segment (start 76.2 35.56) (end 78.0163 35.56) (width 0.8) (layer F.Cu) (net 19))
 (segment (start 78.0163 27.226) (end 78.0163 35.56) (width 0.8) (layer F.Cu) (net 19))
 (segment (start 77.4603 26.67) (end 78.0163 27.226) (width 0.8) (layer F.Cu) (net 19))
 (segment (start 75.66 26.67) (end 77.4603 26.67) (width 0.8) (layer F.Cu) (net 19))
 (segment (start 66.2603 46.99) (end 64.26 46.99) (width 0.8) (layer F.Cu) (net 20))
 (segment (start 66.2603 42.95) (end 66.2603 46.99) (width 0.8) (layer F.Cu) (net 20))
 (segment (start 71.12 38.0903) (end 66.2603 42.95) (width 0.8) (layer F.Cu) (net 20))
 (segment (start 71.12 36.29) (end 71.12 38.0903) (width 0.8) (layer F.Cu) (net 20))
 (segment (start 74.3837 33.02) (end 76.2 33.02) (width 0.8) (layer F.Cu) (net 20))
 (segment (start 72.914 34.4897) (end 74.3837 33.02) (width 0.8) (layer F.Cu) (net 20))
 (segment (start 71.12 34.4897) (end 72.914 34.4897) (width 0.8) (layer F.Cu) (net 20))
 (segment (start 71.12 36.29) (end 71.12 34.4897) (width 0.8) (layer F.Cu) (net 20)))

